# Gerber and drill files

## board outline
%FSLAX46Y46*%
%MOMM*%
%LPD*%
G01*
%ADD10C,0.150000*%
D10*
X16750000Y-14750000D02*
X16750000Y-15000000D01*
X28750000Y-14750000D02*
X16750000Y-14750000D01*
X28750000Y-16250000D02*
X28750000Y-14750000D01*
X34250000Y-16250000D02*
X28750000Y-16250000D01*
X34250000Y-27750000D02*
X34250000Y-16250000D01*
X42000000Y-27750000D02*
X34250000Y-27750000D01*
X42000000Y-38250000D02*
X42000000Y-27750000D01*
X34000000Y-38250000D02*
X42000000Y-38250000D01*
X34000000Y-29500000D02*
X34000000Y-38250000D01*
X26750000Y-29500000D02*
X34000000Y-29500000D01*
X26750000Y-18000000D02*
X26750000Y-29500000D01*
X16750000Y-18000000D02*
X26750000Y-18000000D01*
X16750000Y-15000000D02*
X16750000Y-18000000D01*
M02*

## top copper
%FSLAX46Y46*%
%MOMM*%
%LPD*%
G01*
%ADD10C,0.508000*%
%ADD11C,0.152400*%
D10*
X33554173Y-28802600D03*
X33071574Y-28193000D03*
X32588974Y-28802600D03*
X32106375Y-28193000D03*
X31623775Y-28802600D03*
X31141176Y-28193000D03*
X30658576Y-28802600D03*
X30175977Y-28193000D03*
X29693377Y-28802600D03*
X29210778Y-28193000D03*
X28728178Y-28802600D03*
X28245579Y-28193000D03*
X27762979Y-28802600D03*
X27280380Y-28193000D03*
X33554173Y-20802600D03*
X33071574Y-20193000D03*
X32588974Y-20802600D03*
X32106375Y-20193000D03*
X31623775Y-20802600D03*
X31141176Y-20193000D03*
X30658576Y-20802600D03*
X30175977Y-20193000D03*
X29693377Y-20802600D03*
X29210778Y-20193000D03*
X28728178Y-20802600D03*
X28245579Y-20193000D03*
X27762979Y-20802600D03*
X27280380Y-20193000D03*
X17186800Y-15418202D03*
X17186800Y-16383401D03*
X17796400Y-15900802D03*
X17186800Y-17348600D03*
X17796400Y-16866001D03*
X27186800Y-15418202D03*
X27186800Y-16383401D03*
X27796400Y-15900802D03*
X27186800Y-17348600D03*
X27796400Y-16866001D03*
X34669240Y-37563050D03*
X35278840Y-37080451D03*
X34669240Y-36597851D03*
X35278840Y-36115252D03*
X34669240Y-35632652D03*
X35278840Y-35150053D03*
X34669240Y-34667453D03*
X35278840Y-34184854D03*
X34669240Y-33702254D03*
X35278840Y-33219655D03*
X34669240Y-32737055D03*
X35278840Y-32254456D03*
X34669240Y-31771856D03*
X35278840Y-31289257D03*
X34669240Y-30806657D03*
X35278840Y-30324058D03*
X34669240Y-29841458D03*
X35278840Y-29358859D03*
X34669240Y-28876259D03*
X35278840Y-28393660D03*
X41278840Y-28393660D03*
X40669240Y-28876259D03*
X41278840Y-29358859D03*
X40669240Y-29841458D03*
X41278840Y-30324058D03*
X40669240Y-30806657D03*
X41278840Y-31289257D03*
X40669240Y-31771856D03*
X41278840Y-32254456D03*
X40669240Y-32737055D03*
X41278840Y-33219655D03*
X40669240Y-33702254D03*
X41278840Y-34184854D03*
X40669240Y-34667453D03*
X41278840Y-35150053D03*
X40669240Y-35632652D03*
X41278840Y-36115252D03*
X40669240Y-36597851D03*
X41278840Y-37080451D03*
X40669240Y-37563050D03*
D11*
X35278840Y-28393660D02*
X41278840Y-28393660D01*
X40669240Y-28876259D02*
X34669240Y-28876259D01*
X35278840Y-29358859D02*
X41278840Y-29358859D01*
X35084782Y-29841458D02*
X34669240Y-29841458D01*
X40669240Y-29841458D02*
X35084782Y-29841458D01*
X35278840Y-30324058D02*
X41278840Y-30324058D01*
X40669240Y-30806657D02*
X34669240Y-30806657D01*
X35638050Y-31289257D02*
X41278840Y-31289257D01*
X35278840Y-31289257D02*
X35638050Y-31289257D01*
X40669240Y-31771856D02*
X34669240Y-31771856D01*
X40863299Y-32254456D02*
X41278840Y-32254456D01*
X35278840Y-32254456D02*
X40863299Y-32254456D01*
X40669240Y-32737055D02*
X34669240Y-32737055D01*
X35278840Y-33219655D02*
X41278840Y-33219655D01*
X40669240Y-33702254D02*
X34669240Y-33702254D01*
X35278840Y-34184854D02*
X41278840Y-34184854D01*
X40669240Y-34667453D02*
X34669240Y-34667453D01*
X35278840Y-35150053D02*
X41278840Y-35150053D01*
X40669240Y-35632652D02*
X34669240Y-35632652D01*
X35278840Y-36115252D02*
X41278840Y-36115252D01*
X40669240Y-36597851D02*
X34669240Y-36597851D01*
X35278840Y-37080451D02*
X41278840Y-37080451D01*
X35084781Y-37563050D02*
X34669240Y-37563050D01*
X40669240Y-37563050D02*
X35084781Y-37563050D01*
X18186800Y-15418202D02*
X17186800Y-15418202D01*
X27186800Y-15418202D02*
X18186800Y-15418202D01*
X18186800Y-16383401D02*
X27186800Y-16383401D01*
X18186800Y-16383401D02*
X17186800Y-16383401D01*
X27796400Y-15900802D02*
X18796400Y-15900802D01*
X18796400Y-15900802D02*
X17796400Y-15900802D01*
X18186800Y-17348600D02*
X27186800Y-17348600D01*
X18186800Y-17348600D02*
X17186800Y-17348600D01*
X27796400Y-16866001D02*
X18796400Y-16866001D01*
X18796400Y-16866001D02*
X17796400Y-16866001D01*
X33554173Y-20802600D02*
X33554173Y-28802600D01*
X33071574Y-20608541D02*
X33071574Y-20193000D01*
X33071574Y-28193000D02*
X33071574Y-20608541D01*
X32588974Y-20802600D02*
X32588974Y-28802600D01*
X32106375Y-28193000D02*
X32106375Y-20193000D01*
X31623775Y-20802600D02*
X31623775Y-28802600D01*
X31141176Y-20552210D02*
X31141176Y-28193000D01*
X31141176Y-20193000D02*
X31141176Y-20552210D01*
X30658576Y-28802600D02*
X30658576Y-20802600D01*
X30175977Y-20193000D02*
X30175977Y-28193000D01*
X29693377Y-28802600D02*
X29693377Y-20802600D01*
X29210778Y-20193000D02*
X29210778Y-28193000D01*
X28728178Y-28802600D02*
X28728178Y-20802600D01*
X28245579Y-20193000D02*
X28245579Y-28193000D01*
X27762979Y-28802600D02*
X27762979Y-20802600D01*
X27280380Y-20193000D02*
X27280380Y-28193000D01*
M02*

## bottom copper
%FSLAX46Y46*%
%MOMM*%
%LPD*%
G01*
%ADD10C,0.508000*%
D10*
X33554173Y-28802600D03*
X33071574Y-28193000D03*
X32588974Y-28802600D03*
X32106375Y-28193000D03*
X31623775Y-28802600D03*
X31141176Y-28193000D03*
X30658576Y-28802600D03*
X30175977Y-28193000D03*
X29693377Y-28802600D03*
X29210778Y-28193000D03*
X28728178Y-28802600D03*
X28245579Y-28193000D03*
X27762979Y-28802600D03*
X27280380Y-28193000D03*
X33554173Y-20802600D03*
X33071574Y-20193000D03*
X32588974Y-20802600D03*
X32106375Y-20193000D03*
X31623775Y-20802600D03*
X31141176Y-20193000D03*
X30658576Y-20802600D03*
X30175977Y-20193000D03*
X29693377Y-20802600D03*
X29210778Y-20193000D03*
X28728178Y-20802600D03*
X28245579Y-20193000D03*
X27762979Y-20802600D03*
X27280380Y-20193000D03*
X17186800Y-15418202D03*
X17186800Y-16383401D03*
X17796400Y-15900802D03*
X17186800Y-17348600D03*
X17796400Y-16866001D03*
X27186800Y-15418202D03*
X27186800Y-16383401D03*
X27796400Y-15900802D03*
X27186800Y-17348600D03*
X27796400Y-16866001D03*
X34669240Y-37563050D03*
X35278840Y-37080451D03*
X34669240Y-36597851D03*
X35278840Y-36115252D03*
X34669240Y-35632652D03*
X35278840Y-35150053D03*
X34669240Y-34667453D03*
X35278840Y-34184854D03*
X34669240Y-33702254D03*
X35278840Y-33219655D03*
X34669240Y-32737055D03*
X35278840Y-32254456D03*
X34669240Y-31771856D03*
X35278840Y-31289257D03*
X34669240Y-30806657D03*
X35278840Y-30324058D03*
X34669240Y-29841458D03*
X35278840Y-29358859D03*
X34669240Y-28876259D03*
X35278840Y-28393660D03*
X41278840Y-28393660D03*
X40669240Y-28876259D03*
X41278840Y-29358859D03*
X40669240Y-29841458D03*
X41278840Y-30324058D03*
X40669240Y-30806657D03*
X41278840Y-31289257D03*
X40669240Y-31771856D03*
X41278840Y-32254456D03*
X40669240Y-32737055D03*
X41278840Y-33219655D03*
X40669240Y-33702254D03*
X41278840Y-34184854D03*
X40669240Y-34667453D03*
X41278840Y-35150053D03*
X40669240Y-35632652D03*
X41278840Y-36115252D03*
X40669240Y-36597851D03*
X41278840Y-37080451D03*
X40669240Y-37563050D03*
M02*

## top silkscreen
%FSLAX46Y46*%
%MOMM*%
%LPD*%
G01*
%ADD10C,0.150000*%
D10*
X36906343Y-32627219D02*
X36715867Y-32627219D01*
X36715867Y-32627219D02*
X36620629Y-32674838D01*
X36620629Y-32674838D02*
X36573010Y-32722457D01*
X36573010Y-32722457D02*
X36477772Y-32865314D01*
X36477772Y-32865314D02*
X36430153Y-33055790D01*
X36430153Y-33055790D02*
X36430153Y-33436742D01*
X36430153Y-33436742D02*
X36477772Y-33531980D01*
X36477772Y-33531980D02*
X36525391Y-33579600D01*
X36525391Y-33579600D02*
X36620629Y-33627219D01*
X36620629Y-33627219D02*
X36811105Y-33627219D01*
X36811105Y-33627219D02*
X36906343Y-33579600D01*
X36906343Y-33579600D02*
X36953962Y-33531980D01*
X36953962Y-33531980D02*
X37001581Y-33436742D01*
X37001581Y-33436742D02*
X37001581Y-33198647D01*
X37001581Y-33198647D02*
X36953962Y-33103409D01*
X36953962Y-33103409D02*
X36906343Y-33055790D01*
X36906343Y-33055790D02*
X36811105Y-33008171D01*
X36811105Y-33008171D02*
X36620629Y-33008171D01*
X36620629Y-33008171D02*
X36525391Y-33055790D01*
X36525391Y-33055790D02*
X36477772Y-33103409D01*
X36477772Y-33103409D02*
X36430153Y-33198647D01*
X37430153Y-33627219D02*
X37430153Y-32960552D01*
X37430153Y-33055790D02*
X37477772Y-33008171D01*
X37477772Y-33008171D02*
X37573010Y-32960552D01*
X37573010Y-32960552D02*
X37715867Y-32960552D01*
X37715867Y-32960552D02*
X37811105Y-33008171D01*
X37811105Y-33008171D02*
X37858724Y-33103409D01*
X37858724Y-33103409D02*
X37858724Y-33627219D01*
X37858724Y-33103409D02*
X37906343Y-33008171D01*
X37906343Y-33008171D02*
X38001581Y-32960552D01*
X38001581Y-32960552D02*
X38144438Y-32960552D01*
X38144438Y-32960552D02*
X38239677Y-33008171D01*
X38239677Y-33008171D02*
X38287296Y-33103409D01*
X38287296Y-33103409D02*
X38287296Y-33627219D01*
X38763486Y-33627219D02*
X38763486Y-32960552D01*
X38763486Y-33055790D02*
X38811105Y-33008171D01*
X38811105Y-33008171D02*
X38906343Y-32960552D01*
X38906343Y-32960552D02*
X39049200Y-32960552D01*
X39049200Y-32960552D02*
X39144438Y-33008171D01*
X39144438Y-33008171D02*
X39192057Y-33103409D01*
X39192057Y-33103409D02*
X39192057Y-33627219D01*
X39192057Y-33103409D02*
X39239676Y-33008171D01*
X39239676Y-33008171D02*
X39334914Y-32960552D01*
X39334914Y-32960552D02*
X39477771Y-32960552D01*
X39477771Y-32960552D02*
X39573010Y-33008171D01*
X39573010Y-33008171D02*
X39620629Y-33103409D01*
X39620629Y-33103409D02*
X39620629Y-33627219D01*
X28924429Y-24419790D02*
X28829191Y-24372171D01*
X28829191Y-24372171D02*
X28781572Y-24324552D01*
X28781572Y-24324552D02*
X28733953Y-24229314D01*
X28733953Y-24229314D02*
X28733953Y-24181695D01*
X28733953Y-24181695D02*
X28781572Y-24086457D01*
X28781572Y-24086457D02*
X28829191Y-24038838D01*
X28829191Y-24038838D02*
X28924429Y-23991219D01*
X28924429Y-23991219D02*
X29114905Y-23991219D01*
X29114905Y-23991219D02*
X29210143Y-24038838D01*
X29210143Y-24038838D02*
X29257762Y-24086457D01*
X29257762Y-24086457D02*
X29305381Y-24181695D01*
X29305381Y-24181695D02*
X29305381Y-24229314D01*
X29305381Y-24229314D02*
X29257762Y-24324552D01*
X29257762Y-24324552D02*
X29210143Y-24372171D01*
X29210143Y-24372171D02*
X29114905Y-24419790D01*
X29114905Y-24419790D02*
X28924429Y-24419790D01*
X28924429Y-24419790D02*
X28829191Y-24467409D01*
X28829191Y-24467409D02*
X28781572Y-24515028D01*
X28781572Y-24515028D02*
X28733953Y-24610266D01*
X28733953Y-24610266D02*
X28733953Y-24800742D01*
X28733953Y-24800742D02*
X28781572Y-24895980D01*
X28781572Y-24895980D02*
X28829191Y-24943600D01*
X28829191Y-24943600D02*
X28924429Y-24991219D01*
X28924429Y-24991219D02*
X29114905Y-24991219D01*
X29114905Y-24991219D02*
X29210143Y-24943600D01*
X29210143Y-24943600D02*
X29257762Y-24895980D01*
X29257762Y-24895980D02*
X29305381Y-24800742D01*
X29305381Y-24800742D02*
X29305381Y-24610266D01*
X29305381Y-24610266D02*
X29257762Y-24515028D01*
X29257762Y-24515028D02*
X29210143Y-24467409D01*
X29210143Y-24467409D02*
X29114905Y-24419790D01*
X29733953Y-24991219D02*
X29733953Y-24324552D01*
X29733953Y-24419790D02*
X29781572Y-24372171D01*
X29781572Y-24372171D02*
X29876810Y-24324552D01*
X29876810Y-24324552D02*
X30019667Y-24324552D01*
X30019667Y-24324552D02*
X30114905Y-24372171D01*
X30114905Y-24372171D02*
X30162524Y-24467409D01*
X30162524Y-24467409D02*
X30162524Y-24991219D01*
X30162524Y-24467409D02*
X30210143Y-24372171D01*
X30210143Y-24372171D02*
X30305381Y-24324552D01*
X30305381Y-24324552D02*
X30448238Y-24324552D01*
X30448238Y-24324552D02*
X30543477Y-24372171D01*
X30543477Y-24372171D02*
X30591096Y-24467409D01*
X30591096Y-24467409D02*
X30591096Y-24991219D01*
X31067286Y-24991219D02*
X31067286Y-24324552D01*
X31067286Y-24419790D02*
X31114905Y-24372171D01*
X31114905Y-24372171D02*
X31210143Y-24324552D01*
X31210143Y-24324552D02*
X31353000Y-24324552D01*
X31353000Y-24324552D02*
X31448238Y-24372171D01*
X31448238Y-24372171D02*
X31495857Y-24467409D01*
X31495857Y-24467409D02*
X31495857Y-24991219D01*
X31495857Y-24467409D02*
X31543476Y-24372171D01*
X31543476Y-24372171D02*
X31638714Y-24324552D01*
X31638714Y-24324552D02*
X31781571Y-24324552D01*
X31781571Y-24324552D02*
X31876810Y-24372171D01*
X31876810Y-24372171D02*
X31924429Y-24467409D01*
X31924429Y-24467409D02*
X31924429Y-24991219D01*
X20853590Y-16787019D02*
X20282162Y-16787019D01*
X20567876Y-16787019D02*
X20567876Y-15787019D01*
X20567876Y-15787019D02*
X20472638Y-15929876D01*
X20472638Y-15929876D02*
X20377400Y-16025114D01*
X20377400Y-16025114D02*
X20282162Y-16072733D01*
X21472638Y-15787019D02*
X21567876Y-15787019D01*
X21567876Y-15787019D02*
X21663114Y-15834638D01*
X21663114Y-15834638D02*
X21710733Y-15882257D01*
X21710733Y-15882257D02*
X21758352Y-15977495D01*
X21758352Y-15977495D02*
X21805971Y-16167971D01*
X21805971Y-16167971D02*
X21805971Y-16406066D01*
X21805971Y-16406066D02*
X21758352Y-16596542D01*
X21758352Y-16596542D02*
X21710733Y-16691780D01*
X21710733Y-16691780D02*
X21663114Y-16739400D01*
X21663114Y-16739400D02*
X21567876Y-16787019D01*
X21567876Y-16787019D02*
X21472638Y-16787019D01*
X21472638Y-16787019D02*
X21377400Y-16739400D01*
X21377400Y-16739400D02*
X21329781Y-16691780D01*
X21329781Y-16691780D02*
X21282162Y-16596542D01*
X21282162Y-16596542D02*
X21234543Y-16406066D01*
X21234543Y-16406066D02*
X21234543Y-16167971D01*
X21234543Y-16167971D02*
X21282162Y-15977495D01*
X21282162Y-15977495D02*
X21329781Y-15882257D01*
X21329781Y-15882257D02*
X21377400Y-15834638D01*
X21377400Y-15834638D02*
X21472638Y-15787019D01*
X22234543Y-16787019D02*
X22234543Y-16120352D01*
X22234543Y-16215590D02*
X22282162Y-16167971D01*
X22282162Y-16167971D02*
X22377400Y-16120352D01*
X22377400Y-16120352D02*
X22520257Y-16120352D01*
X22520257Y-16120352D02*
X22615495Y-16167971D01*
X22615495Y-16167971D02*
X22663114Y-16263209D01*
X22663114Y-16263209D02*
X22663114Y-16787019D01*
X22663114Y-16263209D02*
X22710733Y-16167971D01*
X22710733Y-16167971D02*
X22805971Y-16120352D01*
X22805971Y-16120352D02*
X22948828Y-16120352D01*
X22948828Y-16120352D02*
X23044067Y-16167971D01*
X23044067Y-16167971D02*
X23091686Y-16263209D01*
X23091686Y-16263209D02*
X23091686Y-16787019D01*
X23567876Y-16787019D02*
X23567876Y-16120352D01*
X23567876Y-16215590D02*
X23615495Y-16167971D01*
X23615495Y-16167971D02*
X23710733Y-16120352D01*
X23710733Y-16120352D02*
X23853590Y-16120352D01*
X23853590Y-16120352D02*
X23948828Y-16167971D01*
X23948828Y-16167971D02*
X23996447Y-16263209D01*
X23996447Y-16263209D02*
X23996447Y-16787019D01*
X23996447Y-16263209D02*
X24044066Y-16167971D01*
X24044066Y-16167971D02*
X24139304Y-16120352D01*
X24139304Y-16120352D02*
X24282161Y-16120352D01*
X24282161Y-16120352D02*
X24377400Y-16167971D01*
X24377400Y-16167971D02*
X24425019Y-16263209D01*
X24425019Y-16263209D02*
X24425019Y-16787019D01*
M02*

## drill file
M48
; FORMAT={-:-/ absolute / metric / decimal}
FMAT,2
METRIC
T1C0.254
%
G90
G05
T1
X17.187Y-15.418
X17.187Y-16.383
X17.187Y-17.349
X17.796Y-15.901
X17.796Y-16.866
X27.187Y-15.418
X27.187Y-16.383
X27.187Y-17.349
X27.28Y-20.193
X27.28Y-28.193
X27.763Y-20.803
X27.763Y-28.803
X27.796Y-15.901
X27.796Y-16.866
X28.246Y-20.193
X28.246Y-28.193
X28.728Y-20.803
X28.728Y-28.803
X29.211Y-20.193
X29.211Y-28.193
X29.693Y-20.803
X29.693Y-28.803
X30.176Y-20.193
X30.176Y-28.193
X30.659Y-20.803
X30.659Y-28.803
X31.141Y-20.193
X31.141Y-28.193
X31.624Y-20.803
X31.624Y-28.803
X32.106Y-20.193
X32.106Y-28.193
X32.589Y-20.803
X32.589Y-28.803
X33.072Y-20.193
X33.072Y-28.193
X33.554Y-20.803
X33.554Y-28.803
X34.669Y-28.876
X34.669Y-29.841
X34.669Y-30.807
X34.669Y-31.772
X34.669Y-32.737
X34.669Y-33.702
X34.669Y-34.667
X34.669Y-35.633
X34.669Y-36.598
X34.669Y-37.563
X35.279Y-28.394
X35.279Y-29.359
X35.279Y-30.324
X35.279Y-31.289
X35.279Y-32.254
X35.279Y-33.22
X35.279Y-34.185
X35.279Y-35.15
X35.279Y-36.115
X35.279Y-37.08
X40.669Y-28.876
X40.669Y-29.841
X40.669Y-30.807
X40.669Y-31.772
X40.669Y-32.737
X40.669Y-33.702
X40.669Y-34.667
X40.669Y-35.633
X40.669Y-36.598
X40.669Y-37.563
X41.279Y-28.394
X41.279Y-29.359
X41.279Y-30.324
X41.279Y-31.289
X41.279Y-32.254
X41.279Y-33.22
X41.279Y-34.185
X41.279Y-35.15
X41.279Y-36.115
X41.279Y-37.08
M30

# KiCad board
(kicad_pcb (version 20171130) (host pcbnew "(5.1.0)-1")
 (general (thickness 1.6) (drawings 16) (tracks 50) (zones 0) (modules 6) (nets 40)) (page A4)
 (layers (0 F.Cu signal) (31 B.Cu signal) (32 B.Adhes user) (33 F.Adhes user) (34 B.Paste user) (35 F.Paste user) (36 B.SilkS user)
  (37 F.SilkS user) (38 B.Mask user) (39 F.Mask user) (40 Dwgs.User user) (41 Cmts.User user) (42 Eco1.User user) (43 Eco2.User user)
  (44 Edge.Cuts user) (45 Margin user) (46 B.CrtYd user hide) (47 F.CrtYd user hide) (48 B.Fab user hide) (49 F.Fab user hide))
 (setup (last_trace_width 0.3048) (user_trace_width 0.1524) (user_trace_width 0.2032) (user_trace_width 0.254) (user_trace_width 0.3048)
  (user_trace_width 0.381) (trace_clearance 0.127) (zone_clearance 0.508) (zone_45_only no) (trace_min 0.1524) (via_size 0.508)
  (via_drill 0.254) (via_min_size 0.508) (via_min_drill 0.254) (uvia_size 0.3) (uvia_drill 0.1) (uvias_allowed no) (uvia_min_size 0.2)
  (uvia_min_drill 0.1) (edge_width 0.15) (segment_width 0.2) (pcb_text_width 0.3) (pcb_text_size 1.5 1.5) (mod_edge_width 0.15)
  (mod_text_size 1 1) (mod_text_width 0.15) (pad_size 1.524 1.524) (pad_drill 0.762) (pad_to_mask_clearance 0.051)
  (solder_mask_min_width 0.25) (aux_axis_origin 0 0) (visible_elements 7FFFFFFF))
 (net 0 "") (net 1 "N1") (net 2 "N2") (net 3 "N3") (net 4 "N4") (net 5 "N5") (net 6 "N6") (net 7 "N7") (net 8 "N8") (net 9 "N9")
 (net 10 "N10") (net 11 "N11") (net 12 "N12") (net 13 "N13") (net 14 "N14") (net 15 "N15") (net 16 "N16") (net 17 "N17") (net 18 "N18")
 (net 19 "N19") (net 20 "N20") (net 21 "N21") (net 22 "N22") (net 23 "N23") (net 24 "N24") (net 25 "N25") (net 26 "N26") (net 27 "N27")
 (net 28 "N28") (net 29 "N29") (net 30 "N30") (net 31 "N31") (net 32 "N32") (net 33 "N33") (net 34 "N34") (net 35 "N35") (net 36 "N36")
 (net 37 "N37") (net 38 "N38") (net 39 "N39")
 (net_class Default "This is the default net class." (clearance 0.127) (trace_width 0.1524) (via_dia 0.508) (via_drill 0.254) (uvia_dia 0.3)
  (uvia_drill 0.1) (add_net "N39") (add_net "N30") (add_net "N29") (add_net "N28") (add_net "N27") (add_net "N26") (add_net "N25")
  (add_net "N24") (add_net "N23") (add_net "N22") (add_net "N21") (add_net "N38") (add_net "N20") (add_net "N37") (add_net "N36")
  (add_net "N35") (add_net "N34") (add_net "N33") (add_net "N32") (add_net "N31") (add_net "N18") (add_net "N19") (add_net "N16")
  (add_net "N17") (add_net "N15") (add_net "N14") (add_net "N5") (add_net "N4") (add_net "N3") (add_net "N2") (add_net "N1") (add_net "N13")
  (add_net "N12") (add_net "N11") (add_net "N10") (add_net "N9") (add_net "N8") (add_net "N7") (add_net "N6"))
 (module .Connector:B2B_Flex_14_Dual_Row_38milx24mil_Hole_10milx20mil (layer F.Cu) (at 27.28038 28.193)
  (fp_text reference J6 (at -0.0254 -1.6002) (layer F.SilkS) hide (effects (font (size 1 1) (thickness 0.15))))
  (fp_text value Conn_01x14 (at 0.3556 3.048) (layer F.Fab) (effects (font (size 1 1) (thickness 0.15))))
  (pad 14 thru_hole circle (at 6.273793 0.6096) (size 0.508 0.508) (drill 0.254) (layers *.Cu *.Mask) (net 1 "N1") (zone_connect 0))
  (pad 13 thru_hole circle (at 5.791194 0) (size 0.508 0.508) (drill 0.254) (layers *.Cu *.Mask) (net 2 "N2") (zone_connect 0))
  (pad 12 thru_hole circle (at 5.308594 0.6096) (size 0.508 0.508) (drill 0.254) (layers *.Cu *.Mask) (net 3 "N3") (zone_connect 0))
  (pad 11 thru_hole circle (at 4.825995 0) (size 0.508 0.508) (drill 0.254) (layers *.Cu *.Mask) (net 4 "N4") (zone_connect 0))
  (pad 10 thru_hole circle (at 4.343395 0.6096) (size 0.508 0.508) (drill 0.254) (layers *.Cu *.Mask) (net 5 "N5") (zone_connect 0))
  (pad 9 thru_hole circle (at 3.860796 0) (size 0.508 0.508) (drill 0.254) (layers *.Cu *.Mask) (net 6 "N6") (zone_connect 0))
  (pad 8 thru_hole circle (at 3.378196 0.6096) (size 0.508 0.508) (drill 0.254) (layers *.Cu *.Mask) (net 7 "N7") (zone_connect 0))
  (pad 7 thru_hole circle (at 2.895597 0) (size 0.508 0.508) (drill 0.254) (layers *.Cu *.Mask) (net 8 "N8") (zone_connect 0))
  (pad 6 thru_hole circle (at 2.412997 0.6096) (size 0.508 0.508) (drill 0.254) (layers *.Cu *.Mask) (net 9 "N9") (zone_connect 0))
  (pad 5 thru_hole circle (at 1.930398 0) (size 0.508 0.508) (drill 0.254) (layers *.Cu *.Mask) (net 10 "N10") (zone_connect 0))
  (pad 4 thru_hole circle (at 1.447798 0.6096) (size 0.508 0.508) (drill 0.254) (layers *.Cu *.Mask) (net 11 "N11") (zone_connect 0))
  (pad 3 thru_hole circle (at 0.965199 0) (size 0.508 0.508) (drill 0.254) (layers *.Cu *.Mask) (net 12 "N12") (zone_connect 0))
  (pad 2 thru_hole circle (at 0.482599 0.6096) (size 0.508 0.508) (drill 0.254) (layers *.Cu *.Mask) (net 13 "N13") (zone_connect 0))
  (pad 1 thru_hole circle (at 0 0) (size 0.508 0.508) (drill 0.254) (layers *.Cu *.Mask) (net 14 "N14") (zone_connect 0)))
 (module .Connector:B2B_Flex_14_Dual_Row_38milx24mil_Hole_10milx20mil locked (layer F.Cu) (at 27.28038 20.193)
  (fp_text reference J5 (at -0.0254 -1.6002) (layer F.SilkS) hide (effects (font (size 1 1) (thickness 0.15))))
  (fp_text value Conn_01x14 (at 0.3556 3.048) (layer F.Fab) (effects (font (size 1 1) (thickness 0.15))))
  (pad 14 thru_hole circle (at 6.273793 0.6096) (size 0.508 0.508) (drill 0.254) (layers *.Cu *.Mask) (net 1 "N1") (zone_connect 0))
  (pad 13 thru_hole circle (at 5.791194 0) (size 0.508 0.508) (drill 0.254) (layers *.Cu *.Mask) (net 2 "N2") (zone_connect 0))
  (pad 12 thru_hole circle (at 5.308594 0.6096) (size 0.508 0.508) (drill 0.254) (layers *.Cu *.Mask) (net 3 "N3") (zone_connect 0))
  (pad 11 thru_hole circle (at 4.825995 0) (size 0.508 0.508) (drill 0.254) (layers *.Cu *.Mask) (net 4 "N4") (zone_connect 0))
  (pad 10 thru_hole circle (at 4.343395 0.6096) (size 0.508 0.508) (drill 0.254) (layers *.Cu *.Mask) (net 5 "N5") (zone_connect 0))
  (pad 9 thru_hole circle (at 3.860796 0) (size 0.508 0.508) (drill 0.254) (layers *.Cu *.Mask) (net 6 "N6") (zone_connect 0))
  (pad 8 thru_hole circle (at 3.378196 0.6096) (size 0.508 0.508) (drill 0.254) (layers *.Cu *.Mask) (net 7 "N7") (zone_connect 0))
  (pad 7 thru_hole circle (at 2.895597 0) (size 0.508 0.508) (drill 0.254) (layers *.Cu *.Mask) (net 8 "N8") (zone_connect 0))
  (pad 6 thru_hole circle (at 2.412997 0.6096) (size 0.508 0.508) (drill 0.254) (layers *.Cu *.Mask) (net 9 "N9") (zone_connect 0))
  (pad 5 thru_hole circle (at 1.930398 0) (size 0.508 0.508) (drill 0.254) (layers *.Cu *.Mask) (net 10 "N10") (zone_connect 0))
  (pad 4 thru_hole circle (at 1.447798 0.6096) (size 0.508 0.508) (drill 0.254) (layers *.Cu *.Mask) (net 11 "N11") (zone_connect 0))
  (pad 3 thru_hole circle (at 0.965199 0) (size 0.508 0.508) (drill 0.254) (layers *.Cu *.Mask) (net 12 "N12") (zone_connect 0))
  (pad 2 thru_hole circle (at 0.482599 0.6096) (size 0.508 0.508) (drill 0.254) (layers *.Cu *.Mask) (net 13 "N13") (zone_connect 0))
  (pad 1 thru_hole circle (at 0 0) (size 0.508 0.508) (drill 0.254) (layers *.Cu *.Mask) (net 14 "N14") (zone_connect 0)))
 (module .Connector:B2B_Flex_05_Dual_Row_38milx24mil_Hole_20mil (layer F.Cu) (at 17.2118 17.3736 90)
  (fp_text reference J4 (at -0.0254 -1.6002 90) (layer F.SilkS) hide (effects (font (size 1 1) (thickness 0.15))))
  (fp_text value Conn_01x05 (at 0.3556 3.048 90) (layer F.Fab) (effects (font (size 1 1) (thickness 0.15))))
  (pad 5 thru_hole circle (at 1.955398 -0.025 90) (size 0.508 0.508) (drill 0.254) (layers *.Cu *.Mask) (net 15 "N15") (zone_connect 0))
  (pad 3 thru_hole circle (at 0.990199 -0.025 90) (size 0.508 0.508) (drill 0.254) (layers *.Cu *.Mask) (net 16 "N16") (zone_connect 0))
  (pad 4 thru_hole circle (at 1.472798 0.5846 90) (size 0.508 0.508) (drill 0.254) (layers *.Cu *.Mask) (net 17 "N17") (zone_connect 0))
  (pad 1 thru_hole circle (at 0.025 -0.025 90) (size 0.508 0.508) (drill 0.254) (layers *.Cu *.Mask) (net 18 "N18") (zone_connect 0))
  (pad 2 thru_hole circle (at 0.507599 0.5846 90) (size 0.508 0.508) (drill 0.254) (layers *.Cu *.Mask) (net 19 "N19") (zone_connect 0)))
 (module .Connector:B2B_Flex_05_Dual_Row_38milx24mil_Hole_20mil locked (layer F.Cu) (at 27.2118 17.3736 90)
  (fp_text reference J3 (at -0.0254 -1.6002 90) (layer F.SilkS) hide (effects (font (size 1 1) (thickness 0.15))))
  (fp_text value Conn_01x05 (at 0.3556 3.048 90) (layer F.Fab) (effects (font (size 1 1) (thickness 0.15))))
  (pad 5 thru_hole circle (at 1.955398 -0.025 90) (size 0.508 0.508) (drill 0.254) (layers *.Cu *.Mask) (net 15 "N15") (zone_connect 0))
  (pad 3 thru_hole circle (at 0.990199 -0.025 90) (size 0.508 0.508) (drill 0.254) (layers *.Cu *.Mask) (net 16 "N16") (zone_connect 0))
  (pad 4 thru_hole circle (at 1.472798 0.5846 90) (size 0.508 0.508) (drill 0.254) (layers *.Cu *.Mask) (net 17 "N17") (zone_connect 0))
  (pad 1 thru_hole circle (at 0.025 -0.025 90) (size 0.508 0.508) (drill 0.254) (layers *.Cu *.Mask) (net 18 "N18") (zone_connect 0))
  (pad 2 thru_hole circle (at 0.507599 0.5846 90) (size 0.508 0.508) (drill 0.254) (layers *.Cu *.Mask) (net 19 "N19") (zone_connect 0)))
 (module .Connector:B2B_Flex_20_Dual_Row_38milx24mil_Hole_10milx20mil (layer F.Cu) (at 35.27884 28.39366 270)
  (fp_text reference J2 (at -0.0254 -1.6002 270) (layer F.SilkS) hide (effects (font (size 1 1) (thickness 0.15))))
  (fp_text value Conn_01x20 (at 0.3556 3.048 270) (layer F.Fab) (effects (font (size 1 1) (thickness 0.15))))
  (pad 20 thru_hole circle (at 9.16939 0.6096 270) (size 0.508 0.508) (drill 0.254) (layers *.Cu *.Mask) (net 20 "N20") (zone_connect 0))
  (pad 19 thru_hole circle (at 8.686791 0 270) (size 0.508 0.508) (drill 0.254) (layers *.Cu *.Mask) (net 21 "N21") (zone_connect 0))
  (pad 18 thru_hole circle (at 8.204191 0.6096 270) (size 0.508 0.508) (drill 0.254) (layers *.Cu *.Mask) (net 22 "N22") (zone_connect 0))
  (pad 17 thru_hole circle (at 7.721592 0 270) (size 0.508 0.508) (drill 0.254) (layers *.Cu *.Mask) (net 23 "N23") (zone_connect 0))
  (pad 16 thru_hole circle (at 7.238992 0.6096 270) (size 0.508 0.508) (drill 0.254) (layers *.Cu *.Mask) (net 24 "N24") (zone_connect 0))
  (pad 15 thru_hole circle (at 6.756393 0 270) (size 0.508 0.508) (drill 0.254) (layers *.Cu *.Mask) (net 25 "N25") (zone_connect 0))
  (pad 14 thru_hole circle (at 6.273793 0.6096 270) (size 0.508 0.508) (drill 0.254) (layers *.Cu *.Mask) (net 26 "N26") (zone_connect 0))
  (pad 13 thru_hole circle (at 5.791194 0 270) (size 0.508 0.508) (drill 0.254) (layers *.Cu *.Mask) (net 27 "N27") (zone_connect 0))
  (pad 12 thru_hole circle (at 5.308594 0.6096 270) (size 0.508 0.508) (drill 0.254) (layers *.Cu *.Mask) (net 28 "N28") (zone_connect 0))
  (pad 11 thru_hole circle (at 4.825995 0 270) (size 0.508 0.508) (drill 0.254) (layers *.Cu *.Mask) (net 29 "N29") (zone_connect 0))
  (pad 10 thru_hole circle (at 4.343395 0.6096 270) (size 0.508 0.508) (drill 0.254) (layers *.Cu *.Mask) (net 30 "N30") (zone_connect 0))
  (pad 9 thru_hole circle (at 3.860796 0 270) (size 0.508 0.508) (drill 0.254) (layers *.Cu *.Mask) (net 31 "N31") (zone_connect 0))
  (pad 8 thru_hole circle (at 3.378196 0.6096 270) (size 0.508 0.508) (drill 0.254) (layers *.Cu *.Mask) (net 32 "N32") (zone_connect 0))
  (pad 7 thru_hole circle (at 2.895597 0 270) (size 0.508 0.508) (drill 0.254) (layers *.Cu *.Mask) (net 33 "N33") (zone_connect 0))
  (pad 6 thru_hole circle (at 2.412997 0.6096 270) (size 0.508 0.508) (drill 0.254) (layers *.Cu *.Mask) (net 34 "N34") (zone_connect 0))
  (pad 5 thru_hole circle (at 1.930398 0 270) (size 0.508 0.508) (drill 0.254) (layers *.Cu *.Mask) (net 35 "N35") (zone_connect 0))
  (pad 4 thru_hole circle (at 1.447798 0.6096 270) (size 0.508 0.508) (drill 0.254) (layers *.Cu *.Mask) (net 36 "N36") (zone_connect 0))
  (pad 3 thru_hole circle (at 0.965199 0 270) (size 0.508 0.508) (drill 0.254) (layers *.Cu *.Mask) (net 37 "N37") (zone_connect 0))
  (pad 2 thru_hole circle (at 0.482599 0.6096 270) (size 0.508 0.508) (drill 0.254) (layers *.Cu *.Mask) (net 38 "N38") (zone_connect 0))
  (pad 1 thru_hole circle (at 0 0 270) (size 0.508 0.508) (drill 0.254) (layers *.Cu *.Mask) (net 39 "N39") (zone_connect 0)))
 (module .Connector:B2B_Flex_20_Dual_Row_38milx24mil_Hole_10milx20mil (layer F.Cu) (at 41.27884 28.39366 270)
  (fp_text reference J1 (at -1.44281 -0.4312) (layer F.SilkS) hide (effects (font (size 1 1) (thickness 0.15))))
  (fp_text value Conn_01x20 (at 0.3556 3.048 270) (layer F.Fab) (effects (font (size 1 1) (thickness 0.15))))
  (pad 1 thru_hole circle (at 0 0 270) (size 0.508 0.508) (drill 0.254) (layers *.Cu *.Mask) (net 39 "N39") (zone_connect 0))
  (pad 2 thru_hole circle (at 0.482599 0.6096 270) (size 0.508 0.508) (drill 0.254) (layers *.Cu *.Mask) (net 38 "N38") (zone_connect 0))
  (pad 3 thru_hole circle (at 0.965199 0 270) (size 0.508 0.508) (drill 0.254) (layers *.Cu *.Mask) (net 37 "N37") (zone_connect 0))
  (pad 4 thru_hole circle (at 1.447798 0.6096 270) (size 0.508 0.508) (drill 0.254) (layers *.Cu *.Mask) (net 36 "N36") (zone_connect 0))
  (pad 5 thru_hole circle (at 1.930398 0 270) (size 0.508 0.508) (drill 0.254) (layers *.Cu *.Mask) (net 35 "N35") (zone_connect 0))
  (pad 6 thru_hole circle (at 2.412997 0.6096 270) (size 0.508 0.508) (drill 0.254) (layers *.Cu *.Mask) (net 34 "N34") (zone_connect 0))
  (pad 7 thru_hole circle (at 2.895597 0 270) (size 0.508 0.508) (drill 0.254) (layers *.Cu *.Mask) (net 33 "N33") (zone_connect 0))
  (pad 8 thru_hole circle (at 3.378196 0.6096 270) (size 0.508 0.508) (drill 0.254) (layers *.Cu *.Mask) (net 32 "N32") (zone_connect 0))
  (pad 9 thru_hole circle (at 3.860796 0 270) (size 0.508 0.508) (drill 0.254) (layers *.Cu *.Mask) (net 31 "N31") (zone_connect 0))
  (pad 10 thru_hole circle (at 4.343395 0.6096 270) (size 0.508 0.508) (drill 0.254) (layers *.Cu *.Mask) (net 30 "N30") (zone_connect 0))
  (pad 11 thru_hole circle (at 4.825995 0 270) (size 0.508 0.508) (drill 0.254) (layers *.Cu *.Mask) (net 29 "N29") (zone_connect 0))
  (pad 12 thru_hole circle (at 5.308594 0.6096 270) (size 0.508 0.508) (drill 0.254) (layers *.Cu *.Mask) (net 28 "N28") (zone_connect 0))
  (pad 13 thru_hole circle (at 5.791194 0 270) (size 0.508 0.508) (drill 0.254) (layers *.Cu *.Mask) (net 27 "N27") (zone_connect 0))
  (pad 14 thru_hole circle (at 6.273793 0.6096 270) (size 0.508 0.508) (drill 0.254) (layers *.Cu *.Mask) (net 26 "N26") (zone_connect 0))
  (pad 15 thru_hole circle (at 6.756393 0 270) (size 0.508 0.508) (drill 0.254) (layers *.Cu *.Mask) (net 25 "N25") (zone_connect 0))
  (pad 16 thru_hole circle (at 7.238992 0.6096 270) (size 0.508 0.508) (drill 0.254) (layers *.Cu *.Mask) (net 24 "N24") (zone_connect 0))
  (pad 17 thru_hole circle (at 7.721592 0 270) (size 0.508 0.508) (drill 0.254) (layers *.Cu *.Mask) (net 23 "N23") (zone_connect 0))
  (pad 18 thru_hole circle (at 8.204191 0.6096 270) (size 0.508 0.508) (drill 0.254) (layers *.Cu *.Mask) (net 22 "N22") (zone_connect 0))
  (pad 19 thru_hole circle (at 8.686791 0 270) (size 0.508 0.508) (drill 0.254) (layers *.Cu *.Mask) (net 21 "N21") (zone_connect 0))
  (pad 20 thru_hole circle (at 9.16939 0.6096 270) (size 0.508 0.508) (drill 0.254) (layers *.Cu *.Mask) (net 20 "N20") (zone_connect 0)))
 (gr_line (start 16.75 14.75) (end 16.75 15) (layer Edge.Cuts) (width 0.15))
 (gr_line (start 28.75 14.75) (end 16.75 14.75) (layer Edge.Cuts) (width 0.15))
 (gr_line (start 28.75 16.25) (end 28.75 14.75) (layer Edge.Cuts) (width 0.15))
 (gr_line (start 34.25 16.25) (end 28.75 16.25) (layer Edge.Cuts) (width 0.15))
 (gr_line (start 34.25 27.75) (end 34.25 16.25) (layer Edge.Cuts) (width 0.15))
 (gr_line (start 42 27.75) (end 34.25 27.75) (layer Edge.Cuts) (width 0.15))
 (gr_line (start 42 38.25) (end 42 27.75) (layer Edge.Cuts) (width 0.15))
 (gr_line (start 34 38.25) (end 42 38.25) (layer Edge.Cuts) (width 0.15))
 (gr_line (start 34 29.5) (end 34 38.25) (layer Edge.Cuts) (width 0.15))
 (gr_line (start 26.75 29.5) (end 34 29.5) (layer Edge.Cuts) (width 0.15))
 (gr_line (start 26.75 18) (end 26.75 29.5) (layer Edge.Cuts) (width 0.15))
 (gr_line (start 16.75 18) (end 26.75 18) (layer Edge.Cuts) (width 0.15))
 (gr_line (start 16.75 15) (end 16.75 18) (layer Edge.Cuts) (width 0.15))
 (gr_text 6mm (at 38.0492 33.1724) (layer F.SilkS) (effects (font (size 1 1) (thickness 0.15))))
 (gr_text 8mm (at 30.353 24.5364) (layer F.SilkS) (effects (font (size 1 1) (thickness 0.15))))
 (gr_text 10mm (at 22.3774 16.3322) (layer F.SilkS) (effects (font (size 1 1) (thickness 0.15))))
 (segment (start 35.27884 28.39366) (end 41.27884 28.39366) (width 0.1524) (layer F.Cu) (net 39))
 (segment (start 40.66924 28.876259) (end 34.66924 28.876259) (width 0.1524) (layer F.Cu) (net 38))
 (segment (start 35.27884 29.358859) (end 41.27884 29.358859) (width 0.1524) (layer F.Cu) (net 37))
 (segment (start 35.084782 29.841458) (end 34.66924 29.841458) (width 0.1524) (layer F.Cu) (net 36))
 (segment (start 40.66924 29.841458) (end 35.084782 29.841458) (width 0.1524) (layer F.Cu) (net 36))
 (segment (start 35.27884 30.324058) (end 41.27884 30.324058) (width 0.1524) (layer F.Cu) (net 35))
 (segment (start 40.66924 30.806657) (end 34.66924 30.806657) (width 0.1524) (layer F.Cu) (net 34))
 (segment (start 35.63805 31.289257) (end 41.27884 31.289257) (width 0.1524) (layer F.Cu) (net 33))
 (segment (start 35.27884 31.289257) (end 35.63805 31.289257) (width 0.1524) (layer F.Cu) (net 33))
 (segment (start 40.66924 31.771856) (end 34.66924 31.771856) (width 0.1524) (layer F.Cu) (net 32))
 (segment (start 40.863299 32.254456) (end 41.27884 32.254456) (width 0.1524) (layer F.Cu) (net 31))
 (segment (start 35.27884 32.254456) (end 40.863299 32.254456) (width 0.1524) (layer F.Cu) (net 31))
 (segment (start 40.66924 32.737055) (end 34.66924 32.737055) (width 0.1524) (layer F.Cu) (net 30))
 (segment (start 35.27884 33.219655) (end 41.27884 33.219655) (width 0.1524) (layer F.Cu) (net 29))
 (segment (start 40.66924 33.702254) (end 34.66924 33.702254) (width 0.1524) (layer F.Cu) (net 28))
 (segment (start 35.27884 34.184854) (end 41.27884 34.184854) (width 0.1524) (layer F.Cu) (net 27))
 (segment (start 40.66924 34.667453) (end 34.66924 34.667453) (width 0.1524) (layer F.Cu) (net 26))
 (segment (start 35.27884 35.150053) (end 41.27884 35.150053) (width 0.1524) (layer F.Cu) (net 25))
 (segment (start 40.66924 35.632652) (end 34.66924 35.632652) (width 0.1524) (layer F.Cu) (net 24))
 (segment (start 35.27884 36.115252) (end 41.27884 36.115252) (width 0.1524) (layer F.Cu) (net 23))
 (segment (start 40.66924 36.597851) (end 34.66924 36.597851) (width 0.1524) (layer F.Cu) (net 22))
 (segment (start 35.27884 37.080451) (end 41.27884 37.080451) (width 0.1524) (layer F.Cu) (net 21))
 (segment (start 35.084781 37.56305) (end 34.66924 37.56305) (width 0.1524) (layer F.Cu) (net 20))
 (segment (start 40.66924 37.56305) (end 35.084781 37.56305) (width 0.1524) (layer F.Cu) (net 20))
 (segment (start 18.1868 15.418202) (end 17.1868 15.418202) (width 0.1524) (layer F.Cu) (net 15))
 (segment (start 27.1868 15.418202) (end 18.1868 15.418202) (width 0.1524) (layer F.Cu) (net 15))
 (segment (start 18.1868 16.383401) (end 27.1868 16.383401) (width 0.1524) (layer F.Cu) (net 16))
 (segment (start 18.1868 16.383401) (end 17.1868 16.383401) (width 0.1524) (layer F.Cu) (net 16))
 (segment (start 27.7964 15.900802) (end 18.7964 15.900802) (width 0.1524) (layer F.Cu) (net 17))
 (segment (start 18.7964 15.900802) (end 17.7964 15.900802) (width 0.1524) (layer F.Cu) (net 17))
 (segment (start 18.1868 17.3486) (end 27.1868 17.3486) (width 0.1524) (layer F.Cu) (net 18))
 (segment (start 18.1868 17.3486) (end 17.1868 17.3486) (width 0.1524) (layer F.Cu) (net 18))
 (segment (start 27.7964 16.866001) (end 18.7964 16.866001) (width 0.1524) (layer F.Cu) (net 19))
 (segment (start 18.7964 16.866001) (end 17.7964 16.866001) (width 0.1524) (layer F.Cu) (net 19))
 (segment (start 33.554173 20.8026) (end 33.554173 28.8026) (width 0.1524) (layer F.Cu) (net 1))
 (segment (start 33.071574 20.608541) (end 33.071574 20.193) (width 0.1524) (layer F.Cu) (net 2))
 (segment (start 33.071574 28.193) (end 33.071574 20.608541) (width 0.1524) (layer F.Cu) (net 2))
 (segment (start 32.588974 20.8026) (end 32.588974 28.8026) (width 0.1524) (layer F.Cu) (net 3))
 (segment (start 32.106375 28.193) (end 32.106375 20.193) (width 0.1524) (layer F.Cu) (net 4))
 (segment (start 31.623775 20.8026) (end 31.623775 28.8026) (width 0.1524) (layer F.Cu) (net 5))
 (segment (start 31.141176 20.55221) (end 31.141176 28.193) (width 0.1524) (layer F.Cu) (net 6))
 (segment (start 31.141176 20.193) (end 31.141176 20.55221) (width 0.1524) (layer F.Cu) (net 6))
 (segment (start 30.658576 28.8026) (end 30.658576 20.8026) (width 0.1524) (layer F.Cu) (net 7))
 (segment (start 30.175977 20.193) (end 30.175977 28.193) (width 0.1524) (layer F.Cu) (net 8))
 (segment (start 29.693377 28.8026) (end 29.693377 20.8026) (width 0.1524) (layer F.Cu) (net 9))
 (segment (start 29.210778 20.193) (end 29.210778 28.193) (width 0.1524) (layer F.Cu) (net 10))
 (segment (start 28.728178 28.8026) (end 28.728178 20.8026) (width 0.1524) (layer F.Cu) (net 11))
 (segment (start 28.245579 20.193) (end 28.245579 28.193) (width 0.1524) (layer F.Cu) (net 12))
 (segment (start 27.762979 28.8026) (end 27.762979 20.8026) (width 0.1524) (layer F.Cu) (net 13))
 (segment (start 27.28038 20.193) (end 27.28038 28.193) (width 0.1524) (layer F.Cu) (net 14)))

